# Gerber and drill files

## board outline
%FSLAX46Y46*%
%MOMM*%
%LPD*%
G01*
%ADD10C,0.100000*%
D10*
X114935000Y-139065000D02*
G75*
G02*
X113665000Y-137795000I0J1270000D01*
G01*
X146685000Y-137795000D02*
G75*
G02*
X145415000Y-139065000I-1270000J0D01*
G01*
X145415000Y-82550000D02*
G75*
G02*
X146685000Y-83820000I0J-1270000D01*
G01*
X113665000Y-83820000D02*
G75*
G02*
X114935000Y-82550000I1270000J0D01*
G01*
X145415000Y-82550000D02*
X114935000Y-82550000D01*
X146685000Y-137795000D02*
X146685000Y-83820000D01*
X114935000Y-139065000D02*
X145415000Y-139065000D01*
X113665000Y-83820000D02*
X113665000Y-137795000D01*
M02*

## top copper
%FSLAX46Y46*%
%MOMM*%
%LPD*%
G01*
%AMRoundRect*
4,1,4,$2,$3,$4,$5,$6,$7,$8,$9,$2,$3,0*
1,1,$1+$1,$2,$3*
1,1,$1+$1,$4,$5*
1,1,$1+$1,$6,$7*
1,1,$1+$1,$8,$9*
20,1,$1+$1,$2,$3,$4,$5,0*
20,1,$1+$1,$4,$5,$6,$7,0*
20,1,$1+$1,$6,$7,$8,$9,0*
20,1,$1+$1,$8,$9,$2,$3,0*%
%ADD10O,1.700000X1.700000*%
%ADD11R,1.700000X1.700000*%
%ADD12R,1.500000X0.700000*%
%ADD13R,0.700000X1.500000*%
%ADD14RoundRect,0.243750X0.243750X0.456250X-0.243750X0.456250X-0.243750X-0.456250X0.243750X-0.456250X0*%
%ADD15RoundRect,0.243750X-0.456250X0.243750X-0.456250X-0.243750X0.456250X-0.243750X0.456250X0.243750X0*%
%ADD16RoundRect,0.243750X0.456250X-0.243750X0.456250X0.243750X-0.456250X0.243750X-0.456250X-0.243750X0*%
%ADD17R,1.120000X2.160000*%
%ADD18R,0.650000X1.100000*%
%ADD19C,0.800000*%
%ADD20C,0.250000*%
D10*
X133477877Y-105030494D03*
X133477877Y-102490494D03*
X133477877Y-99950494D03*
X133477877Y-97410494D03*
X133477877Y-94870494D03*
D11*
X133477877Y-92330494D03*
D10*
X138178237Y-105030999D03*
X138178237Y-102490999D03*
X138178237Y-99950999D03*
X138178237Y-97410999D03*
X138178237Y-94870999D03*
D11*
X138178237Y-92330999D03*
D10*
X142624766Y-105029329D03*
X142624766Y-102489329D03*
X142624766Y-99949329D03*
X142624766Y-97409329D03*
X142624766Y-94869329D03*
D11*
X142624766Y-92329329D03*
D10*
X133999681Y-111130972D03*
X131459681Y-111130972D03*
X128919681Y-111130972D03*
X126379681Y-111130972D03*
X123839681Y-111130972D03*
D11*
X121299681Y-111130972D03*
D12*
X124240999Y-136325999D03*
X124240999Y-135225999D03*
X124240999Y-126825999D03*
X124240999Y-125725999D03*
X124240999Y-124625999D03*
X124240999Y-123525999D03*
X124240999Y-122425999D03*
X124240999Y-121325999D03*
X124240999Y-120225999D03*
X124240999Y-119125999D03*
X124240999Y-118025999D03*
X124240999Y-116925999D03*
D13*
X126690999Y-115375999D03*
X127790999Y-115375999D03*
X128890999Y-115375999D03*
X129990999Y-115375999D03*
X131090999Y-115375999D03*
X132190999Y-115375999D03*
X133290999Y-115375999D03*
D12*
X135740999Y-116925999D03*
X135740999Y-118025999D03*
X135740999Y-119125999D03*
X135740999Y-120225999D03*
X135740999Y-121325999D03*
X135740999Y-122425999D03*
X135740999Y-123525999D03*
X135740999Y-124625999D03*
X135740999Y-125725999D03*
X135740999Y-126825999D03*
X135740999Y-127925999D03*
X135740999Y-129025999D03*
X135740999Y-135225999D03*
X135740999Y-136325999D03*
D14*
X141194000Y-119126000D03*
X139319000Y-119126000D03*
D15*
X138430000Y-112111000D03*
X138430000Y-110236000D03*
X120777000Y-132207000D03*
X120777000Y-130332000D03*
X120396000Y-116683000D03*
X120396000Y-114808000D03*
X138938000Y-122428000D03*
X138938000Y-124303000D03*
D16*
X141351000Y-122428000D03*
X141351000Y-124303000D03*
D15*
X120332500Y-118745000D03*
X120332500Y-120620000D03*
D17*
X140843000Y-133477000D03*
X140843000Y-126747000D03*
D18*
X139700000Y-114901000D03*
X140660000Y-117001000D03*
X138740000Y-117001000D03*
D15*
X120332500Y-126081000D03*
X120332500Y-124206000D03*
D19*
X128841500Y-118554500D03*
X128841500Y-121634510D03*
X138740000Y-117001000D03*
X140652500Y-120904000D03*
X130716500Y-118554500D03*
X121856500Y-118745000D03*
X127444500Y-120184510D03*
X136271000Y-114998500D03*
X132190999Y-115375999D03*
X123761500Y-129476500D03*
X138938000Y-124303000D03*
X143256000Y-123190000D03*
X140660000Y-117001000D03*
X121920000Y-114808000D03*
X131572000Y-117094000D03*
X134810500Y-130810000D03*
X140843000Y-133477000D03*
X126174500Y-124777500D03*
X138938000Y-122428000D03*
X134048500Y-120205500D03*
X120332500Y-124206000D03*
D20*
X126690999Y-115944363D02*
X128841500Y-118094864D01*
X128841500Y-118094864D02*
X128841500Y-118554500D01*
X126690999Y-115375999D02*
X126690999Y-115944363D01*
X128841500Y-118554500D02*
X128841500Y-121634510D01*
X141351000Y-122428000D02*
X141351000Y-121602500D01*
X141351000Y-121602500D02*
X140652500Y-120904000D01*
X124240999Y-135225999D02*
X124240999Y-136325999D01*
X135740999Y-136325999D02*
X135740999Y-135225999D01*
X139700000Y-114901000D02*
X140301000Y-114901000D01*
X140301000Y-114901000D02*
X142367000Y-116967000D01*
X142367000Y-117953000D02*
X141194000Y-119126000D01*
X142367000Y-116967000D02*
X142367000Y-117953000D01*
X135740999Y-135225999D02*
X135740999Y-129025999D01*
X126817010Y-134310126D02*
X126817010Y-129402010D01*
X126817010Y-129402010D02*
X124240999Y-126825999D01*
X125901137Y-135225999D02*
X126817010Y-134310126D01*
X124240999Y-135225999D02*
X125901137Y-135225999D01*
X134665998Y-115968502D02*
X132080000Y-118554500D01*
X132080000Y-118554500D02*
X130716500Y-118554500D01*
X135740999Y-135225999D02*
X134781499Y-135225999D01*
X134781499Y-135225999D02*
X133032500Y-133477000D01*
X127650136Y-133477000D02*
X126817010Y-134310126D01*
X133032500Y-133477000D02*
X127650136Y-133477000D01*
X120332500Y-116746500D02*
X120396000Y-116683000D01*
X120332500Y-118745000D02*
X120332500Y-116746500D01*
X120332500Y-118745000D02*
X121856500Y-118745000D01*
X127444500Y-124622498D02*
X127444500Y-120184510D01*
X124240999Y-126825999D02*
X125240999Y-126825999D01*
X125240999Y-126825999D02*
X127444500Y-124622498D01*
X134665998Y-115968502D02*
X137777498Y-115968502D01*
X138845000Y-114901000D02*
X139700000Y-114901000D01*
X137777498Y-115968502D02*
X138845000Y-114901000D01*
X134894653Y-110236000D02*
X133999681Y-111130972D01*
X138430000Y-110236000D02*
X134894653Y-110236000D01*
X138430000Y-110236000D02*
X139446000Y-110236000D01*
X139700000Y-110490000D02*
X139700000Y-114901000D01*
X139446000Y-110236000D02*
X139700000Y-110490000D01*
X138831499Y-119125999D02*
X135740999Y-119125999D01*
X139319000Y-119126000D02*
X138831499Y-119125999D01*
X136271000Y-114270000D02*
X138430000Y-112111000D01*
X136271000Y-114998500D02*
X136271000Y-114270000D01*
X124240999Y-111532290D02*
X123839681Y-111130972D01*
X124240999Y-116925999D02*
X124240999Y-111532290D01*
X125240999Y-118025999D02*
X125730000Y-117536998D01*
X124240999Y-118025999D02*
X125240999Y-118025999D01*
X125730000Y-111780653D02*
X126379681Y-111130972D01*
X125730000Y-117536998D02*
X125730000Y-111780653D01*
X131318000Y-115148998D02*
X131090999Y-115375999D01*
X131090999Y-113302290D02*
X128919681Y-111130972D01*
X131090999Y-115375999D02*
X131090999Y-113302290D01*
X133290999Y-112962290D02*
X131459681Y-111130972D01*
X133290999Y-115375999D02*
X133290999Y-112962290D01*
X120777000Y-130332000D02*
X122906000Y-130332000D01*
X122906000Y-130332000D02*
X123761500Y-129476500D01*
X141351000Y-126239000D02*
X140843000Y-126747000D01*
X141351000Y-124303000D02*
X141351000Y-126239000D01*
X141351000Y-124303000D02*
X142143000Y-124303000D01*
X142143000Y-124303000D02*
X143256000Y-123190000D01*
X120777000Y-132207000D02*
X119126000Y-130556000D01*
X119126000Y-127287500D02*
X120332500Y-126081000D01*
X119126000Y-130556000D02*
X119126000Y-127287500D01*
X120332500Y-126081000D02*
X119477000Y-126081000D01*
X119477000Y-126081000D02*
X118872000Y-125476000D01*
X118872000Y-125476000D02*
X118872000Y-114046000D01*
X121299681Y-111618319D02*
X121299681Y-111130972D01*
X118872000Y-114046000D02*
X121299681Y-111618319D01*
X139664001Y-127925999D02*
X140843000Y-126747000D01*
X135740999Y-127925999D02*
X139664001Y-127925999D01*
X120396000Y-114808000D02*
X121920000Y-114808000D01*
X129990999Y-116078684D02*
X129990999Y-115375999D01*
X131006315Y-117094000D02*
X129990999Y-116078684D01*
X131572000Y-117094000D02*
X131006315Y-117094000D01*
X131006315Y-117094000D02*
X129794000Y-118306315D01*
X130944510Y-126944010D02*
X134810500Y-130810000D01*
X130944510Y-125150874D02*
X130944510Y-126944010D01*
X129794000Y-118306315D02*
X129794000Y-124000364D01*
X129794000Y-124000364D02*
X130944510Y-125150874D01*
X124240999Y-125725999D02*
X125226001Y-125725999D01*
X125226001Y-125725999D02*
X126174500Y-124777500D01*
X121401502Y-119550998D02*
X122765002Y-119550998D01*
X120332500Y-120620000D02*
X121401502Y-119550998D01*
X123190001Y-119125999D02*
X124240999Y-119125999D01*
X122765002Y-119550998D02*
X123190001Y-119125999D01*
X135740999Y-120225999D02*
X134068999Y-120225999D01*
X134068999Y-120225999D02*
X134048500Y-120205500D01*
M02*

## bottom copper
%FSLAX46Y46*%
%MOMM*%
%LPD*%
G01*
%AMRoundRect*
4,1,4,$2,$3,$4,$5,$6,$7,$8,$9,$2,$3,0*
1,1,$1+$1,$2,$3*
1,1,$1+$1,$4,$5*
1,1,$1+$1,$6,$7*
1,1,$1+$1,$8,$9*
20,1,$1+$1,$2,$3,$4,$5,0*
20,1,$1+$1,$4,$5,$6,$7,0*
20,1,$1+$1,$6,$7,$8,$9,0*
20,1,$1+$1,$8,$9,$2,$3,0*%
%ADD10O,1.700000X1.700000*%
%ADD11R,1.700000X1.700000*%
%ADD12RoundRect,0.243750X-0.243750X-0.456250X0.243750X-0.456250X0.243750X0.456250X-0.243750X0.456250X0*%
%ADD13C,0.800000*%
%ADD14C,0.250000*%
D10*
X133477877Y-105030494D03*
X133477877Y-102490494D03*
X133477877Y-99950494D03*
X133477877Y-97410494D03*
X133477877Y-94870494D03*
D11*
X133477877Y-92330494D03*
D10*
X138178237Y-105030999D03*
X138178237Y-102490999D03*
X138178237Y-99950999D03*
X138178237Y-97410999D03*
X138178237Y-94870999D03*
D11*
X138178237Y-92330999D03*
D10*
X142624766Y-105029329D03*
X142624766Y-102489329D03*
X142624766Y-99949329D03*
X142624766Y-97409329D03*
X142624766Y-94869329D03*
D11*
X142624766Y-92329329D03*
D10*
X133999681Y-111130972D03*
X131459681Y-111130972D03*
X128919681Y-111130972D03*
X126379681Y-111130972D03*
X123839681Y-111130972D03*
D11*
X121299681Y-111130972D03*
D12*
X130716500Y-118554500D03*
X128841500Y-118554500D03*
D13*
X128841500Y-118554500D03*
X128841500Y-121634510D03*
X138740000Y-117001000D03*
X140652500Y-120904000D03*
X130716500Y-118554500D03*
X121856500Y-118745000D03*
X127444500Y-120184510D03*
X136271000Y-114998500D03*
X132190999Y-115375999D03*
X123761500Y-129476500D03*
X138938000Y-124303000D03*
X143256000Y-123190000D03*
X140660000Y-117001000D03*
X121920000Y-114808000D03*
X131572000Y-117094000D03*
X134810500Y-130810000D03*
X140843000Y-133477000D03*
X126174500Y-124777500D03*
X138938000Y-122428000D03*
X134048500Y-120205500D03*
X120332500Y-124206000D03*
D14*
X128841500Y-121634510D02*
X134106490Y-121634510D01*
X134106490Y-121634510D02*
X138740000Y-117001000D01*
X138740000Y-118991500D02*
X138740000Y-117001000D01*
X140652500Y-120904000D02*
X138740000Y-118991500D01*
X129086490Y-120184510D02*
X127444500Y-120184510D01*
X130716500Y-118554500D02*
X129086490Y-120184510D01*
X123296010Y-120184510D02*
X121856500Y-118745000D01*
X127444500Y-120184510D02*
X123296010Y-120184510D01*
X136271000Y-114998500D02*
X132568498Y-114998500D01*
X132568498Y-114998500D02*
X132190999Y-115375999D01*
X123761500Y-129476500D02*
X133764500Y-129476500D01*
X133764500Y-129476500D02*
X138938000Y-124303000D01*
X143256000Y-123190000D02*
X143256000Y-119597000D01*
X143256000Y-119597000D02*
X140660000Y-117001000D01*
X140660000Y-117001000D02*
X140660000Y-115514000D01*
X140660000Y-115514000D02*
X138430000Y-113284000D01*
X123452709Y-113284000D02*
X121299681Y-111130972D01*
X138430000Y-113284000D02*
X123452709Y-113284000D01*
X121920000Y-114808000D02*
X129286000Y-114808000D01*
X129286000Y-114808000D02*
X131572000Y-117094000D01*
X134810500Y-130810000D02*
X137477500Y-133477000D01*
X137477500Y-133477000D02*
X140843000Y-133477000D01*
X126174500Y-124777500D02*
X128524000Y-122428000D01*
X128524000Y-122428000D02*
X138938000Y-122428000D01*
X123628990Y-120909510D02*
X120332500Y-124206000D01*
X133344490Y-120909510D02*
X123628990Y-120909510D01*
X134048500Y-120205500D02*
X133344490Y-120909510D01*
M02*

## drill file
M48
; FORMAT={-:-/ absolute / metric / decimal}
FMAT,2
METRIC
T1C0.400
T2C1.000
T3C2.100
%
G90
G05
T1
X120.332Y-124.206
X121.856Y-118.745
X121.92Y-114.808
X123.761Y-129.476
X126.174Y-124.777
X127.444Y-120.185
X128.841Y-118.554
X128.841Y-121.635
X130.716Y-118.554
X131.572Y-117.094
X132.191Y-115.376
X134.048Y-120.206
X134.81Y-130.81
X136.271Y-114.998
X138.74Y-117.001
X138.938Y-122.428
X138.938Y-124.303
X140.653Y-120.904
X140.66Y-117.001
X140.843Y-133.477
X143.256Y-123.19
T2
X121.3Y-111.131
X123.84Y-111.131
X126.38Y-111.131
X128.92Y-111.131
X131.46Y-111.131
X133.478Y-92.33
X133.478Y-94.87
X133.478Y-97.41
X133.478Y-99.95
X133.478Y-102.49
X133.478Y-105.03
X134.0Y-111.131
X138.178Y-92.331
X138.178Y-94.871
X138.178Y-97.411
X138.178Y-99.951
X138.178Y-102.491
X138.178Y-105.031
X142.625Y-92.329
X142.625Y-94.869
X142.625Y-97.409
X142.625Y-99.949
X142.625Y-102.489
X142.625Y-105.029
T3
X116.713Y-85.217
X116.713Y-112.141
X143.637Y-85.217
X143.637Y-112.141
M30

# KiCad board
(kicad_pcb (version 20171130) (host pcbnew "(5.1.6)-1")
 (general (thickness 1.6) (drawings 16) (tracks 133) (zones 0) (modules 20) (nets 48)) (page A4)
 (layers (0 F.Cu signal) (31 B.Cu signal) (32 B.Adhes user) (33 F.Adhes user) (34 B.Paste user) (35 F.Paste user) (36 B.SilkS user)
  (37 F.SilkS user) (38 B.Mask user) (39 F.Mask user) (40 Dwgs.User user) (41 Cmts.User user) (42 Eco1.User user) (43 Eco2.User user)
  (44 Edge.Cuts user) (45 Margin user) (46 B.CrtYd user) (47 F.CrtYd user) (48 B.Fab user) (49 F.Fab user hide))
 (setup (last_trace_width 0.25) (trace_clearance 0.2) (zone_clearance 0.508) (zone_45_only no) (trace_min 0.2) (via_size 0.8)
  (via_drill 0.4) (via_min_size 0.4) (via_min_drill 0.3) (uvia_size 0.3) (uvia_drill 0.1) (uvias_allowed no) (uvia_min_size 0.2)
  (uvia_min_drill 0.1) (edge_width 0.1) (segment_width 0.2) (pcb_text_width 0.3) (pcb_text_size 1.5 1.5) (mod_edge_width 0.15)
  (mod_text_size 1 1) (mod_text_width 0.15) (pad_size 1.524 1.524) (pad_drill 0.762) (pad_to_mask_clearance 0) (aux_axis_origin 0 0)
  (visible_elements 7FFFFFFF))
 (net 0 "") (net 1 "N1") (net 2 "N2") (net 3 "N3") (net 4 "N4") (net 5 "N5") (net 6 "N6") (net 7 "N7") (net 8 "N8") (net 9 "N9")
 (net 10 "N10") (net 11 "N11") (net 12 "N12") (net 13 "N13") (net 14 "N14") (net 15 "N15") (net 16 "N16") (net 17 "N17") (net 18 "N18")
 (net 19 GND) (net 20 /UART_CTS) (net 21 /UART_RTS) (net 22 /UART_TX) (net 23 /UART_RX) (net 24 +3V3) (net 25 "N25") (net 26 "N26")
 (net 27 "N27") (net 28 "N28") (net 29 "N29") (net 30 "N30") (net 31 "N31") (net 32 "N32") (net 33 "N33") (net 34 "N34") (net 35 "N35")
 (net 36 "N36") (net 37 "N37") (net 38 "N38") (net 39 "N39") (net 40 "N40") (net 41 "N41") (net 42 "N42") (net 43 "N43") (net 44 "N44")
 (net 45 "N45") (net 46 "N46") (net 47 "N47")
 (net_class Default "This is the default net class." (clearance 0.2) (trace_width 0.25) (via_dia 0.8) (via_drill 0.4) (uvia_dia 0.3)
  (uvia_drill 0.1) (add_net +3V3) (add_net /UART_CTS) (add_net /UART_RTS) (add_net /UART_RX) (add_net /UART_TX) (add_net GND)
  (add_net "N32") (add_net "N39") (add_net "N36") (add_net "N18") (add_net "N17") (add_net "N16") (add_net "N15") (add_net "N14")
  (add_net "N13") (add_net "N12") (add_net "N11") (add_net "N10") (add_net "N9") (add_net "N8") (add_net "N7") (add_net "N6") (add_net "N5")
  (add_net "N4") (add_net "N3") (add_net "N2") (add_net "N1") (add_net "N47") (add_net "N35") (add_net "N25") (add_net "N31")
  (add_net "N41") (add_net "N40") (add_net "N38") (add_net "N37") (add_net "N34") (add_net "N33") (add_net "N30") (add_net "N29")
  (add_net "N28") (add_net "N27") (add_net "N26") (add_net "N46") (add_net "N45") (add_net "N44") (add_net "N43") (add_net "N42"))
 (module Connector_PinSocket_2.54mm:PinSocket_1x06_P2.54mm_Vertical (layer B.Cu) (at 133.477877 92.330494 180)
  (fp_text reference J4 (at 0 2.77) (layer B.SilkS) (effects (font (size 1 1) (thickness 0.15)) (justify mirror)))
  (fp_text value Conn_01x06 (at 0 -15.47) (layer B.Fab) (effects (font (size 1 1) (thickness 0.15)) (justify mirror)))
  (pad 6 thru_hole oval (at 0 -12.7 180) (size 1.7 1.7) (drill 1) (layers *.Cu *.Mask) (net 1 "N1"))
  (pad 5 thru_hole oval (at 0 -10.16 180) (size 1.7 1.7) (drill 1) (layers *.Cu *.Mask) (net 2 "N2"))
  (pad 4 thru_hole oval (at 0 -7.62 180) (size 1.7 1.7) (drill 1) (layers *.Cu *.Mask) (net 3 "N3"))
  (pad 3 thru_hole oval (at 0 -5.08 180) (size 1.7 1.7) (drill 1) (layers *.Cu *.Mask) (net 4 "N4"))
  (pad 2 thru_hole oval (at 0 -2.54 180) (size 1.7 1.7) (drill 1) (layers *.Cu *.Mask) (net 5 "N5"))
  (pad 1 thru_hole rect (at 0 0 180) (size 1.7 1.7) (drill 1) (layers *.Cu *.Mask) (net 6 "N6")))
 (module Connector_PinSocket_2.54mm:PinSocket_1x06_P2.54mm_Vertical (layer B.Cu) (at 138.178237 92.330999 180)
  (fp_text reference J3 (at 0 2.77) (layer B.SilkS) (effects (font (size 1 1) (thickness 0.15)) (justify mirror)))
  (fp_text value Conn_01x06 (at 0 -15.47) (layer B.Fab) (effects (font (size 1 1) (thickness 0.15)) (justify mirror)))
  (pad 6 thru_hole oval (at 0 -12.7 180) (size 1.7 1.7) (drill 1) (layers *.Cu *.Mask) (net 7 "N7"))
  (pad 5 thru_hole oval (at 0 -10.16 180) (size 1.7 1.7) (drill 1) (layers *.Cu *.Mask) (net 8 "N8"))
  (pad 4 thru_hole oval (at 0 -7.62 180) (size 1.7 1.7) (drill 1) (layers *.Cu *.Mask) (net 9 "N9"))
  (pad 3 thru_hole oval (at 0 -5.08 180) (size 1.7 1.7) (drill 1) (layers *.Cu *.Mask) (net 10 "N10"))
  (pad 2 thru_hole oval (at 0 -2.54 180) (size 1.7 1.7) (drill 1) (layers *.Cu *.Mask) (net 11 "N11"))
  (pad 1 thru_hole rect (at 0 0 180) (size 1.7 1.7) (drill 1) (layers *.Cu *.Mask) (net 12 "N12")))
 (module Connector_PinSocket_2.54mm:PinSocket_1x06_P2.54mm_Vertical (layer B.Cu) (at 142.624766 92.329329 180)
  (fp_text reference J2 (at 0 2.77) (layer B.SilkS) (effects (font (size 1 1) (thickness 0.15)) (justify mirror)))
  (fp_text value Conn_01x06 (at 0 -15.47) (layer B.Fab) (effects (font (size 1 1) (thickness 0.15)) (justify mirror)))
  (pad 6 thru_hole oval (at 0 -12.7 180) (size 1.7 1.7) (drill 1) (layers *.Cu *.Mask) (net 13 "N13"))
  (pad 5 thru_hole oval (at 0 -10.16 180) (size 1.7 1.7) (drill 1) (layers *.Cu *.Mask) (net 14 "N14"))
  (pad 4 thru_hole oval (at 0 -7.62 180) (size 1.7 1.7) (drill 1) (layers *.Cu *.Mask) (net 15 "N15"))
  (pad 3 thru_hole oval (at 0 -5.08 180) (size 1.7 1.7) (drill 1) (layers *.Cu *.Mask) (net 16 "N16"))
  (pad 2 thru_hole oval (at 0 -2.54 180) (size 1.7 1.7) (drill 1) (layers *.Cu *.Mask) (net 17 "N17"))
  (pad 1 thru_hole rect (at 0 0 180) (size 1.7 1.7) (drill 1) (layers *.Cu *.Mask) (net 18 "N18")))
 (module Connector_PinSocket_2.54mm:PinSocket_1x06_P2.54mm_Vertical (layer B.Cu) (at 121.299681 111.130972 270)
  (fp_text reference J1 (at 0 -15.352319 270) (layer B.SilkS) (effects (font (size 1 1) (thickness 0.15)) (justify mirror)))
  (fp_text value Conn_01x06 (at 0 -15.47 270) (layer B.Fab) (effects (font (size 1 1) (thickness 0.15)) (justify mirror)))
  (pad 6 thru_hole oval (at 0 -12.7 270) (size 1.7 1.7) (drill 1) (layers *.Cu *.Mask) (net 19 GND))
  (pad 5 thru_hole oval (at 0 -10.16 270) (size 1.7 1.7) (drill 1) (layers *.Cu *.Mask) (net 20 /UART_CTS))
  (pad 4 thru_hole oval (at 0 -7.62 270) (size 1.7 1.7) (drill 1) (layers *.Cu *.Mask) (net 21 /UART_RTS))
  (pad 3 thru_hole oval (at 0 -5.08 270) (size 1.7 1.7) (drill 1) (layers *.Cu *.Mask) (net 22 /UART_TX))
  (pad 2 thru_hole oval (at 0 -2.54 270) (size 1.7 1.7) (drill 1) (layers *.Cu *.Mask) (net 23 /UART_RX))
  (pad 1 thru_hole rect (at 0 0 270) (size 1.7 1.7) (drill 1) (layers *.Cu *.Mask) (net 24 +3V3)))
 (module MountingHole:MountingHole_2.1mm (layer F.Cu) (at 143.637 112.141)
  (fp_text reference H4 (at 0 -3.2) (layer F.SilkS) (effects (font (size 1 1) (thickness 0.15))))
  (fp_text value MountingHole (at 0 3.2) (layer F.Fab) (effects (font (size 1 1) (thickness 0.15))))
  (pad "" np_thru_hole circle (at 0 0) (size 2.1 2.1) (drill 2.1) (layers *.Cu *.Mask)))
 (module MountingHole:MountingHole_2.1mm (layer F.Cu) (at 116.713 112.141)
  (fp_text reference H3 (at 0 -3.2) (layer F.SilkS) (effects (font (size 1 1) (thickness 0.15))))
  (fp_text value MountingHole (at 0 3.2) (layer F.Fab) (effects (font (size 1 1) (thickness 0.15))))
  (pad "" np_thru_hole circle (at 0 0) (size 2.1 2.1) (drill 2.1) (layers *.Cu *.Mask)))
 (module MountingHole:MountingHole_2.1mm (layer F.Cu) (at 143.637 85.217)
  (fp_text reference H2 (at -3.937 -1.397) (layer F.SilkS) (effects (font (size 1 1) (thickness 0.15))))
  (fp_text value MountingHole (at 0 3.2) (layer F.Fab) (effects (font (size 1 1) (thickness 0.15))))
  (pad "" np_thru_hole circle (at 0 0) (size 2.1 2.1) (drill 2.1) (layers *.Cu *.Mask)))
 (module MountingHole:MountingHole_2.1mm (layer F.Cu) (at 116.713 85.217)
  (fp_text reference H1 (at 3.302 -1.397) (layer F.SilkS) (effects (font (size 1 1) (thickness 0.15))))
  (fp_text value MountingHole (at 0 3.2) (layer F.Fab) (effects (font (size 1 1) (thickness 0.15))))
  (pad "" np_thru_hole circle (at 0 0) (size 2.1 2.1) (drill 2.1) (layers *.Cu *.Mask)))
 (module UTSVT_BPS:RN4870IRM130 (layer F.Cu) (at 129.990999 126.125999 180)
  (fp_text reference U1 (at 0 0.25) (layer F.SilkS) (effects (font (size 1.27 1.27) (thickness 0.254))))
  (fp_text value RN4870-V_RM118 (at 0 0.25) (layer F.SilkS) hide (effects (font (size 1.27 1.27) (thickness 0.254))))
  (pad 33 smd rect (at 5.75 -10.2 270) (size 0.7 1.5) (layers F.Cu F.Paste F.Mask) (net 19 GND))
  (pad 32 smd rect (at 5.75 -9.1 270) (size 0.7 1.5) (layers F.Cu F.Paste F.Mask) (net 19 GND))
  (pad 31 smd rect (at 5.75 -0.7 270) (size 0.7 1.5) (layers F.Cu F.Paste F.Mask) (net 19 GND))
  (pad 30 smd rect (at 5.75 0.4 270) (size 0.7 1.5) (layers F.Cu F.Paste F.Mask) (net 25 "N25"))
  (pad 29 smd rect (at 5.75 1.5 270) (size 0.7 1.5) (layers F.Cu F.Paste F.Mask) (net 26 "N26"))
  (pad 28 smd rect (at 5.75 2.6 270) (size 0.7 1.5) (layers F.Cu F.Paste F.Mask) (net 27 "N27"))
  (pad 27 smd rect (at 5.75 3.7 270) (size 0.7 1.5) (layers F.Cu F.Paste F.Mask) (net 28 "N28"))
  (pad 26 smd rect (at 5.75 4.8 270) (size 0.7 1.5) (layers F.Cu F.Paste F.Mask) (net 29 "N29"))
  (pad 25 smd rect (at 5.75 5.9 270) (size 0.7 1.5) (layers F.Cu F.Paste F.Mask) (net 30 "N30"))
  (pad 24 smd rect (at 5.75 7 270) (size 0.7 1.5) (layers F.Cu F.Paste F.Mask) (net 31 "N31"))
  (pad 23 smd rect (at 5.75 8.1 270) (size 0.7 1.5) (layers F.Cu F.Paste F.Mask) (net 22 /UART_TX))
  (pad 22 smd rect (at 5.75 9.2 270) (size 0.7 1.5) (layers F.Cu F.Paste F.Mask) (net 23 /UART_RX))
  (pad 21 smd rect (at 3.3 10.75 180) (size 0.7 1.5) (layers F.Cu F.Paste F.Mask) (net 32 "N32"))
  (pad 20 smd rect (at 2.2 10.75 180) (size 0.7 1.5) (layers F.Cu F.Paste F.Mask) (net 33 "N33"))
  (pad 19 smd rect (at 1.1 10.75 180) (size 0.7 1.5) (layers F.Cu F.Paste F.Mask) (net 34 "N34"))
  (pad 18 smd rect (at 0 10.75 180) (size 0.7 1.5) (layers F.Cu F.Paste F.Mask) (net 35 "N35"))
  (pad 17 smd rect (at -1.1 10.75 180) (size 0.7 1.5) (layers F.Cu F.Paste F.Mask) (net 21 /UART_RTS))
  (pad 16 smd rect (at -2.2 10.75 180) (size 0.7 1.5) (layers F.Cu F.Paste F.Mask) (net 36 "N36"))
  (pad 15 smd rect (at -3.3 10.75 180) (size 0.7 1.5) (layers F.Cu F.Paste F.Mask) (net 20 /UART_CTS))
  (pad 14 smd rect (at -5.75 9.2 270) (size 0.7 1.5) (layers F.Cu F.Paste F.Mask) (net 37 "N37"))
  (pad 13 smd rect (at -5.75 8.1 270) (size 0.7 1.5) (layers F.Cu F.Paste F.Mask) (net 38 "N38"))
  (pad 12 smd rect (at -5.75 7 270) (size 0.7 1.5) (layers F.Cu F.Paste F.Mask) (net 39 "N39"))
  (pad 11 smd rect (at -5.75 5.9 270) (size 0.7 1.5) (layers F.Cu F.Paste F.Mask) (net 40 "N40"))
  (pad 10 smd rect (at -5.75 4.8 270) (size 0.7 1.5) (layers F.Cu F.Paste F.Mask) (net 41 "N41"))
  (pad 9 smd rect (at -5.75 3.7 270) (size 0.7 1.5) (layers F.Cu F.Paste F.Mask) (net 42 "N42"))
  (pad 8 smd rect (at -5.75 2.6 270) (size 0.7 1.5) (layers F.Cu F.Paste F.Mask) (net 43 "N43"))
  (pad 7 smd rect (at -5.75 1.5 270) (size 0.7 1.5) (layers F.Cu F.Paste F.Mask) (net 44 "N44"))
  (pad 6 smd rect (at -5.75 0.4 270) (size 0.7 1.5) (layers F.Cu F.Paste F.Mask) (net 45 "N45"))
  (pad 5 smd rect (at -5.75 -0.7 270) (size 0.7 1.5) (layers F.Cu F.Paste F.Mask) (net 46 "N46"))
  (pad 4 smd rect (at -5.75 -1.8 270) (size 0.7 1.5) (layers F.Cu F.Paste F.Mask) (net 24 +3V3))
  (pad 3 smd rect (at -5.75 -2.9 270) (size 0.7 1.5) (layers F.Cu F.Paste F.Mask) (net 19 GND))
  (pad 2 smd rect (at -5.75 -9.1 270) (size 0.7 1.5) (layers F.Cu F.Paste F.Mask) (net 19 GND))
  (pad 1 smd rect (at -5.75 -10.2 270) (size 0.7 1.5) (layers F.Cu F.Paste F.Mask) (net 19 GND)))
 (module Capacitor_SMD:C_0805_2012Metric (layer B.Cu) (at 129.779 118.5545)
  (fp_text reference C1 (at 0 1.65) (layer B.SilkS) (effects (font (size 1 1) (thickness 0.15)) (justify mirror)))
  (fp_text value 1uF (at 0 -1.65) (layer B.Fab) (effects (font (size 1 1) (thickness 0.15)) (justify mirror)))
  (pad 2 smd roundrect (at 0.9375 0) (size 0.975 1.4) (layers B.Cu B.Paste B.Mask) (roundrect_rratio 0.25) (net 19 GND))
  (pad 1 smd roundrect (at -0.9375 0) (size 0.975 1.4) (layers B.Cu B.Paste B.Mask) (roundrect_rratio 0.25) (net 32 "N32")))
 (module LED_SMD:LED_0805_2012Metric (layer F.Cu) (at 140.2565 119.126 180)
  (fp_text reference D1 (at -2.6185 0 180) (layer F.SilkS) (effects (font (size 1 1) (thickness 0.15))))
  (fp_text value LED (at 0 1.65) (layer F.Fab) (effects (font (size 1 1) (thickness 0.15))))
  (pad 1 smd roundrect (at -0.9375 0 180) (size 0.975 1.4) (layers F.Cu F.Paste F.Mask) (roundrect_rratio 0.25) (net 19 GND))
  (pad 2 smd roundrect (at 0.9375 0 180) (size 0.975 1.4) (layers F.Cu F.Paste F.Mask) (roundrect_rratio 0.25) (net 39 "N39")))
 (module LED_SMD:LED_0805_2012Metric (layer F.Cu) (at 138.43 111.1735 270)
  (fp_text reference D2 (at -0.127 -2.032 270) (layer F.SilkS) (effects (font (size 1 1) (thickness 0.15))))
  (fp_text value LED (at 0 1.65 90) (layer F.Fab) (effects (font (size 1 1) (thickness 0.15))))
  (pad 2 smd roundrect (at 0.9375 0 270) (size 0.975 1.4) (layers F.Cu F.Paste F.Mask) (roundrect_rratio 0.25) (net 36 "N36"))
  (pad 1 smd roundrect (at -0.9375 0 270) (size 0.975 1.4) (layers F.Cu F.Paste F.Mask) (roundrect_rratio 0.25) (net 19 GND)))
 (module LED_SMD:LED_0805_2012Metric (layer F.Cu) (at 120.777 131.2695 270)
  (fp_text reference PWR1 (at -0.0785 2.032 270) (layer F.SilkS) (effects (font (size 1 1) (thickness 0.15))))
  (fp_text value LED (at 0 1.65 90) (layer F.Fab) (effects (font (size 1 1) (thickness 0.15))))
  (pad 2 smd roundrect (at 0.9375 0 270) (size 0.975 1.4) (layers F.Cu F.Paste F.Mask) (roundrect_rratio 0.25) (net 24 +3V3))
  (pad 1 smd roundrect (at -0.9375 0 270) (size 0.975 1.4) (layers F.Cu F.Paste F.Mask) (roundrect_rratio 0.25) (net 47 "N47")))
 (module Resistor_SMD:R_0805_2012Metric (layer F.Cu) (at 120.396 115.7455 270)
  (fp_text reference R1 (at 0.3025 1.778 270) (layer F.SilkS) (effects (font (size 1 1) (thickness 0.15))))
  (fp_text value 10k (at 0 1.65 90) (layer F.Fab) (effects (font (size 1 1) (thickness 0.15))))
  (pad 2 smd roundrect (at 0.9375 0 270) (size 0.975 1.4) (layers F.Cu F.Paste F.Mask) (roundrect_rratio 0.25) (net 19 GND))
  (pad 1 smd roundrect (at -0.9375 0 270) (size 0.975 1.4) (layers F.Cu F.Paste F.Mask) (roundrect_rratio 0.25) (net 35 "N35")))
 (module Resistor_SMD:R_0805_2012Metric (layer F.Cu) (at 138.938 123.3655 270)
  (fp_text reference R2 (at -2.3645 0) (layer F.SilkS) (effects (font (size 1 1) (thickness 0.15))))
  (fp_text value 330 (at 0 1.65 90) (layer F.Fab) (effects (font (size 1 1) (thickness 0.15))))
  (pad 1 smd roundrect (at -0.9375 0 270) (size 0.975 1.4) (layers F.Cu F.Paste F.Mask) (roundrect_rratio 0.25) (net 25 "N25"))
  (pad 2 smd roundrect (at 0.9375 0 270) (size 0.975 1.4) (layers F.Cu F.Paste F.Mask) (roundrect_rratio 0.25) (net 47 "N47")))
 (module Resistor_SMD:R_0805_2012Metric (layer F.Cu) (at 141.351 123.3655 90)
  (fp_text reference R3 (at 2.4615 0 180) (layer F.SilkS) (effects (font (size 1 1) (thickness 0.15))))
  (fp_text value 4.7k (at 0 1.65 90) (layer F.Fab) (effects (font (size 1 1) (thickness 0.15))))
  (pad 2 smd roundrect (at 0.9375 0 90) (size 0.975 1.4) (layers F.Cu F.Paste F.Mask) (roundrect_rratio 0.25) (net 32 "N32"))
  (pad 1 smd roundrect (at -0.9375 0 90) (size 0.975 1.4) (layers F.Cu F.Paste F.Mask) (roundrect_rratio 0.25) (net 24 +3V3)))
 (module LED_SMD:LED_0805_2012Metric (layer F.Cu) (at 120.3325 119.6825 270)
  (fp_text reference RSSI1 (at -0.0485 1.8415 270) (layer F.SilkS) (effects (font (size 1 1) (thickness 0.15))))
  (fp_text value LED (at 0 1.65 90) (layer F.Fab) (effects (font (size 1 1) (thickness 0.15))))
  (pad 1 smd roundrect (at -0.9375 0 270) (size 0.975 1.4) (layers F.Cu F.Paste F.Mask) (roundrect_rratio 0.25) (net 19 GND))
  (pad 2 smd roundrect (at 0.9375 0 270) (size 0.975 1.4) (layers F.Cu F.Paste F.Mask) (roundrect_rratio 0.25) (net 31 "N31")))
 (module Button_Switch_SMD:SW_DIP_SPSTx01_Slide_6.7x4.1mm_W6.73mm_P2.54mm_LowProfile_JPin (layer F.Cu) (at 140.843 130.112 270)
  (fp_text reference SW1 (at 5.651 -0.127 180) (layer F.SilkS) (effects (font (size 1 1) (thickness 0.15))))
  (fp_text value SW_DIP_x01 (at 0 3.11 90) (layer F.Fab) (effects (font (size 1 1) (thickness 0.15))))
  (pad 2 smd rect (at 3.365 0 270) (size 2.16 1.12) (layers F.Cu F.Paste F.Mask) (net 35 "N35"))
  (pad 1 smd rect (at -3.365 0 270) (size 2.16 1.12) (layers F.Cu F.Paste F.Mask) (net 24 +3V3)))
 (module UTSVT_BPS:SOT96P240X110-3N (layer F.Cu) (at 139.7 115.951 90)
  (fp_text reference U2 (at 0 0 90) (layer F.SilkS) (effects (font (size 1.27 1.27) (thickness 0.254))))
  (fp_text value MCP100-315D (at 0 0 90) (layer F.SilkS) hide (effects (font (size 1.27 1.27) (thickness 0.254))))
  (pad 3 smd rect (at 1.05 0 180) (size 0.65 1.1) (layers F.Cu F.Paste F.Mask) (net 19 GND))
  (pad 2 smd rect (at -1.05 0.96 180) (size 0.65 1.1) (layers F.Cu F.Paste F.Mask) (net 24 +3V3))
  (pad 1 smd rect (at -1.05 -0.96 180) (size 0.65 1.1) (layers F.Cu F.Paste F.Mask) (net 32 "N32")))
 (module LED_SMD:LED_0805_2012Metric (layer F.Cu) (at 120.3325 125.1435 270)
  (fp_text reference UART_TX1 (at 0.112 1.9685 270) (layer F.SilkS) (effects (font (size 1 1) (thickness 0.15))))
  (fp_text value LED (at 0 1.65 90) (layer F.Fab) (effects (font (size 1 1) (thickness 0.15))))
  (pad 2 smd roundrect (at 0.9375 0 270) (size 0.975 1.4) (layers F.Cu F.Paste F.Mask) (roundrect_rratio 0.25) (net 24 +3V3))
  (pad 1 smd roundrect (at -0.9375 0 270) (size 0.975 1.4) (layers F.Cu F.Paste F.Mask) (roundrect_rratio 0.25) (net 40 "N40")))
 (gr_arc (start 114.935 137.795) (end 113.665 137.795) (angle -90) (layer Edge.Cuts) (width 0.1))
 (gr_arc (start 145.415 137.795) (end 145.415 139.065) (angle -90) (layer Edge.Cuts) (width 0.1))
 (gr_arc (start 145.415 83.82) (end 146.685 83.82) (angle -90) (layer Edge.Cuts) (width 0.1))
 (gr_arc (start 114.935 83.82) (end 114.935 82.55) (angle -90) (layer Edge.Cuts) (width 0.1))
 (gr_line (start 145.415 82.55) (end 114.935 82.55) (layer Edge.Cuts) (width 0.1))
 (gr_line (start 146.685 137.795) (end 146.685 83.82) (layer Edge.Cuts) (width 0.1))
 (gr_line (start 114.935 139.065) (end 145.415 139.065) (layer Edge.Cuts) (width 0.1))
 (gr_line (start 113.665 83.82) (end 113.665 137.795) (layer Edge.Cuts) (width 0.1))
 (via (at 128.8415 118.5545) (size 0.8) (drill 0.4) (layers F.Cu B.Cu) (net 32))
 (segment (start 126.690999 115.944363) (end 128.8415 118.094864) (width 0.25) (layer F.Cu) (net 32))
 (segment (start 128.8415 118.094864) (end 128.8415 118.5545) (width 0.25) (layer F.Cu) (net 32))
 (segment (start 126.690999 115.375999) (end 126.690999 115.944363) (width 0.25) (layer F.Cu) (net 32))
 (via (at 128.8415 121.63451) (size 0.8) (drill 0.4) (layers F.Cu B.Cu) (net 32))
 (segment (start 128.8415 118.5545) (end 128.8415 121.63451) (width 0.25) (layer F.Cu) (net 32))
 (via (at 138.74 117.001) (size 0.8) (drill 0.4) (layers F.Cu B.Cu) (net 32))
 (segment (start 128.8415 121.63451) (end 134.10649 121.63451) (width 0.25) (layer B.Cu) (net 32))
 (segment (start 134.10649 121.63451) (end 138.74 117.001) (width 0.25) (layer B.Cu) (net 32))
 (segment (start 141.351 122.428) (end 141.351 121.6025) (width 0.25) (layer F.Cu) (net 32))
 (via (at 140.6525 120.904) (size 0.8) (drill 0.4) (layers F.Cu B.Cu) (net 32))
 (segment (start 141.351 121.6025) (end 140.6525 120.904) (width 0.25) (layer F.Cu) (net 32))
 (segment (start 138.74 118.9915) (end 138.74 117.001) (width 0.25) (layer B.Cu) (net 32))
 (segment (start 140.6525 120.904) (end 138.74 118.9915) (width 0.25) (layer B.Cu) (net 32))
 (segment (start 124.240999 135.225999) (end 124.240999 136.325999) (width 0.25) (layer F.Cu) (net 19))
 (segment (start 135.740999 136.325999) (end 135.740999 135.225999) (width 0.25) (layer F.Cu) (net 19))
 (segment (start 139.7 114.901) (end 140.301 114.901) (width 0.25) (layer F.Cu) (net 19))
 (segment (start 140.301 114.901) (end 142.367 116.967) (width 0.25) (layer F.Cu) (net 19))
 (segment (start 142.367 117.953) (end 141.194 119.126) (width 0.25) (layer F.Cu) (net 19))
 (segment (start 142.367 116.967) (end 142.367 117.953) (width 0.25) (layer F.Cu) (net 19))
 (segment (start 135.740999 135.225999) (end 135.740999 129.025999) (width 0.25) (layer F.Cu) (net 19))
 (segment (start 126.81701 134.310126) (end 126.81701 129.40201) (width 0.25) (layer F.Cu) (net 19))
 (segment (start 126.81701 129.40201) (end 124.240999 126.825999) (width 0.25) (layer F.Cu) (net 19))
 (segment (start 125.901137 135.225999) (end 126.81701 134.310126) (width 0.25) (layer F.Cu) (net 19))
 (segment (start 124.240999 135.225999) (end 125.901137 135.225999) (width 0.25) (layer F.Cu) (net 19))
 (via (at 130.7165 118.5545) (size 0.8) (drill 0.4) (layers F.Cu B.Cu) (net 19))
 (segment (start 134.665998 115.968502) (end 132.08 118.5545) (width 0.25) (layer F.Cu) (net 19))
 (segment (start 132.08 118.5545) (end 130.7165 118.5545) (width 0.25) (layer F.Cu) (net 19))
 (segment (start 135.740999 135.225999) (end 134.781499 135.225999) (width 0.25) (layer F.Cu) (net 19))
 (segment (start 134.781499 135.225999) (end 133.0325 133.477) (width 0.25) (layer F.Cu) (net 19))
 (segment (start 127.650136 133.477) (end 126.81701 134.310126) (width 0.25) (layer F.Cu) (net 19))
 (segment (start 133.0325 133.477) (end 127.650136 133.477) (width 0.25) (layer F.Cu) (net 19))
 (segment (start 120.3325 116.7465) (end 120.396 116.683) (width 0.25) (layer F.Cu) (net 19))
 (segment (start 120.3325 118.745) (end 120.3325 116.7465) (width 0.25) (layer F.Cu) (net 19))
 (via (at 121.8565 118.745) (size 0.8) (drill 0.4) (layers F.Cu B.Cu) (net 19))
 (segment (start 120.3325 118.745) (end 121.8565 118.745) (width 0.25) (layer F.Cu) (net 19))
 (via (at 127.4445 120.18451) (size 0.8) (drill 0.4) (layers F.Cu B.Cu) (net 19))
 (segment (start 127.4445 124.622498) (end 127.4445 120.18451) (width 0.25) (layer F.Cu) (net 19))
 (segment (start 124.240999 126.825999) (end 125.240999 126.825999) (width 0.25) (layer F.Cu) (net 19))
 (segment (start 125.240999 126.825999) (end 127.4445 124.622498) (width 0.25) (layer F.Cu) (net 19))
 (segment (start 129.08649 120.18451) (end 127.4445 120.18451) (width 0.25) (layer B.Cu) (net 19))
 (segment (start 130.7165 118.5545) (end 129.08649 120.18451) (width 0.25) (layer B.Cu) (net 19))
 (segment (start 123.29601 120.18451) (end 121.8565 118.745) (width 0.25) (layer B.Cu) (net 19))
 (segment (start 127.4445 120.18451) (end 123.29601 120.18451) (width 0.25) (layer B.Cu) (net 19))
 (segment (start 134.665998 115.968502) (end 137.777498 115.968502) (width 0.25) (layer F.Cu) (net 19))
 (segment (start 138.845 114.901) (end 139.7 114.901) (width 0.25) (layer F.Cu) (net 19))
 (segment (start 137.777498 115.968502) (end 138.845 114.901) (width 0.25) (layer F.Cu) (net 19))
 (segment (start 134.894653 110.236) (end 133.999681 111.130972) (width 0.25) (layer F.Cu) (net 19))
 (segment (start 138.43 110.236) (end 134.894653 110.236) (width 0.25) (layer F.Cu) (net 19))
 (segment (start 138.43 110.236) (end 139.446 110.236) (width 0.25) (layer F.Cu) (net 19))
 (segment (start 139.7 110.49) (end 139.7 114.901) (width 0.25) (layer F.Cu) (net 19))
 (segment (start 139.446 110.236) (end 139.7 110.49) (width 0.25) (layer F.Cu) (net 19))
 (segment (start 138.831499 119.125999) (end 135.740999 119.125999) (width 0.25) (layer F.Cu) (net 39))
 (segment (start 139.319 119.126) (end 138.831499 119.125999) (width 0.25) (layer F.Cu) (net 39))
 (via (at 136.271 114.9985) (size 0.8) (drill 0.4) (layers F.Cu B.Cu) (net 36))
 (via (at 132.190999 115.375999) (size 0.8) (drill 0.4) (layers F.Cu B.Cu) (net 36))
 (segment (start 136.271 114.9985) (end 132.568498 114.9985) (width 0.25) (layer B.Cu) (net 36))
 (segment (start 132.568498 114.9985) (end 132.190999 115.375999) (width 0.25) (layer B.Cu) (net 36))
 (segment (start 136.271 114.27) (end 138.43 112.111) (width 0.25) (layer F.Cu) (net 36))
 (segment (start 136.271 114.9985) (end 136.271 114.27) (width 0.25) (layer F.Cu) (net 36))
 (segment (start 124.240999 111.53229) (end 123.839681 111.130972) (width 0.25) (layer F.Cu) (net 23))
 (segment (start 124.240999 116.925999) (end 124.240999 111.53229) (width 0.25) (layer F.Cu) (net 23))
 (segment (start 125.240999 118.025999) (end 125.73 117.536998) (width 0.25) (layer F.Cu) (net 22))
 (segment (start 124.240999 118.025999) (end 125.240999 118.025999) (width 0.25) (layer F.Cu) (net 22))
 (segment (start 125.73 111.780653) (end 126.379681 111.130972) (width 0.25) (layer F.Cu) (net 22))
 (segment (start 125.73 117.536998) (end 125.73 111.780653) (width 0.25) (layer F.Cu) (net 22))
 (segment (start 131.318 115.148998) (end 131.090999 115.375999) (width 0.25) (layer F.Cu) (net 21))
 (segment (start 131.090999 113.30229) (end 128.919681 111.130972) (width 0.25) (layer F.Cu) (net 21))
 (segment (start 131.090999 115.375999) (end 131.090999 113.30229) (width 0.25) (layer F.Cu) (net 21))
 (segment (start 133.290999 112.96229) (end 131.459681 111.130972) (width 0.25) (layer F.Cu) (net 20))
 (segment (start 133.290999 115.375999) (end 133.290999 112.96229) (width 0.25) (layer F.Cu) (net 20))
 (via (at 123.7615 129.4765) (size 0.8) (drill 0.4) (layers F.Cu B.Cu) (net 47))
 (segment (start 120.777 130.332) (end 122.906 130.332) (width 0.25) (layer F.Cu) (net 47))
 (segment (start 122.906 130.332) (end 123.7615 129.4765) (width 0.25) (layer F.Cu) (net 47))
 (via (at 138.938 124.303) (size 0.8) (drill 0.4) (layers F.Cu B.Cu) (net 47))
 (segment (start 123.7615 129.4765) (end 133.7645 129.4765) (width 0.25) (layer B.Cu) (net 47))
 (segment (start 133.7645 129.4765) (end 138.938 124.303) (width 0.25) (layer B.Cu) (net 47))
 (segment (start 141.351 126.239) (end 140.843 126.747) (width 0.25) (layer F.Cu) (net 24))
 (segment (start 141.351 124.303) (end 141.351 126.239) (width 0.25) (layer F.Cu) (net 24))
 (via (at 143.256 123.19) (size 0.8) (drill 0.4) (layers F.Cu B.Cu) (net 24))
 (segment (start 141.351 124.303) (end 142.143 124.303) (width 0.25) (layer F.Cu) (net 24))
 (segment (start 142.143 124.303) (end 143.256 123.19) (width 0.25) (layer F.Cu) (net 24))
 (segment (start 120.777 132.207) (end 119.126 130.556) (width 0.25) (layer F.Cu) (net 24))
 (segment (start 119.126 127.2875) (end 120.3325 126.081) (width 0.25) (layer F.Cu) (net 24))
 (segment (start 119.126 130.556) (end 119.126 127.2875) (width 0.25) (layer F.Cu) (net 24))
 (via (at 140.66 117.001) (size 0.8) (drill 0.4) (layers F.Cu B.Cu) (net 24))
 (segment (start 143.256 123.19) (end 143.256 119.597) (width 0.25) (layer B.Cu) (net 24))
 (segment (start 143.256 119.597) (end 140.66 117.001) (width 0.25) (layer B.Cu) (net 24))
 (segment (start 140.66 117.001) (end 140.66 115.514) (width 0.25) (layer B.Cu) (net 24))
 (segment (start 140.66 115.514) (end 138.43 113.284) (width 0.25) (layer B.Cu) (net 24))
 (segment (start 123.452709 113.284) (end 121.299681 111.130972) (width 0.25) (layer B.Cu) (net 24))
 (segment (start 138.43 113.284) (end 123.452709 113.284) (width 0.25) (layer B.Cu) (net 24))
 (segment (start 120.3325 126.081) (end 119.477 126.081) (width 0.25) (layer F.Cu) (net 24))
 (segment (start 119.477 126.081) (end 118.872 125.476) (width 0.25) (layer F.Cu) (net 24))
 (segment (start 118.872 125.476) (end 118.872 114.046) (width 0.25) (layer F.Cu) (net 24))
 (segment (start 121.299681 111.618319) (end 121.299681 111.130972) (width 0.25) (layer F.Cu) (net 24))
 (segment (start 118.872 114.046) (end 121.299681 111.618319) (width 0.25) (layer F.Cu) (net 24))
 (segment (start 139.664001 127.925999) (end 140.843 126.747) (width 0.25) (layer F.Cu) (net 24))
 (segment (start 135.740999 127.925999) (end 139.664001 127.925999) (width 0.25) (layer F.Cu) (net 24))
 (via (at 121.92 114.808) (size 0.8) (drill 0.4) (layers F.Cu B.Cu) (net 35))
 (segment (start 120.396 114.808) (end 121.92 114.808) (width 0.25) (layer F.Cu) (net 35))
 (via (at 131.572 117.094) (size 0.8) (drill 0.4) (layers F.Cu B.Cu) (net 35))
 (segment (start 121.92 114.808) (end 129.286 114.808) (width 0.25) (layer B.Cu) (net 35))
 (segment (start 129.286 114.808) (end 131.572 117.094) (width 0.25) (layer B.Cu) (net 35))
 (segment (start 129.990999 116.078684) (end 129.990999 115.375999) (width 0.25) (layer F.Cu) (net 35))
 (segment (start 131.006315 117.094) (end 129.990999 116.078684) (width 0.25) (layer F.Cu) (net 35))
 (segment (start 131.572 117.094) (end 131.006315 117.094) (width 0.25) (layer F.Cu) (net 35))
 (segment (start 131.006315 117.094) (end 129.794 118.306315) (width 0.25) (layer F.Cu) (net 35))
 (via (at 134.8105 130.81) (size 0.8) (drill 0.4) (layers F.Cu B.Cu) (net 35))
 (segment (start 130.94451 126.94401) (end 134.8105 130.81) (width 0.25) (layer F.Cu) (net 35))
 (segment (start 130.94451 125.150874) (end 130.94451 126.94401) (width 0.25) (layer F.Cu) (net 35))
 (segment (start 129.794 118.306315) (end 129.794 124.000364) (width 0.25) (layer F.Cu) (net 35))
 (segment (start 129.794 124.000364) (end 130.94451 125.150874) (width 0.25) (layer F.Cu) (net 35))
 (via (at 140.843 133.477) (size 0.8) (drill 0.4) (layers F.Cu B.Cu) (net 35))
 (segment (start 134.8105 130.81) (end 137.4775 133.477) (width 0.25) (layer B.Cu) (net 35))
 (segment (start 137.4775 133.477) (end 140.843 133.477) (width 0.25) (layer B.Cu) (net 35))
 (via (at 126.1745 124.7775) (size 0.8) (drill 0.4) (layers F.Cu B.Cu) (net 25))
 (segment (start 124.240999 125.725999) (end 125.226001 125.725999) (width 0.25) (layer F.Cu) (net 25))
 (segment (start 125.226001 125.725999) (end 126.1745 124.7775) (width 0.25) (layer F.Cu) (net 25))
 (via (at 138.938 122.428) (size 0.8) (drill 0.4) (layers F.Cu B.Cu) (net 25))
 (segment (start 126.1745 124.7775) (end 128.524 122.428) (width 0.25) (layer B.Cu) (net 25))
 (segment (start 128.524 122.428) (end 138.938 122.428) (width 0.25) (layer B.Cu) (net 25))
 (segment (start 121.401502 119.550998) (end 122.765002 119.550998) (width 0.25) (layer F.Cu) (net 31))
 (segment (start 120.3325 120.62) (end 121.401502 119.550998) (width 0.25) (layer F.Cu) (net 31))
 (segment (start 123.190001 119.125999) (end 124.240999 119.125999) (width 0.25) (layer F.Cu) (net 31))
 (segment (start 122.765002 119.550998) (end 123.190001 119.125999) (width 0.25) (layer F.Cu) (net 31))
 (via (at 134.0485 120.2055) (size 0.8) (drill 0.4) (layers F.Cu B.Cu) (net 40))
 (segment (start 135.740999 120.225999) (end 134.068999 120.225999) (width 0.25) (layer F.Cu) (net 40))
 (segment (start 134.068999 120.225999) (end 134.0485 120.2055) (width 0.25) (layer F.Cu) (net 40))
 (via (at 120.3325 124.206) (size 0.8) (drill 0.4) (layers F.Cu B.Cu) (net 40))
 (segment (start 123.62899 120.90951) (end 120.3325 124.206) (width 0.25) (layer B.Cu) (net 40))
 (segment (start 133.34449 120.90951) (end 123.62899 120.90951) (width 0.25) (layer B.Cu) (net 40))
 (segment (start 134.0485 120.2055) (end 133.34449 120.90951) (width 0.25) (layer B.Cu) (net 40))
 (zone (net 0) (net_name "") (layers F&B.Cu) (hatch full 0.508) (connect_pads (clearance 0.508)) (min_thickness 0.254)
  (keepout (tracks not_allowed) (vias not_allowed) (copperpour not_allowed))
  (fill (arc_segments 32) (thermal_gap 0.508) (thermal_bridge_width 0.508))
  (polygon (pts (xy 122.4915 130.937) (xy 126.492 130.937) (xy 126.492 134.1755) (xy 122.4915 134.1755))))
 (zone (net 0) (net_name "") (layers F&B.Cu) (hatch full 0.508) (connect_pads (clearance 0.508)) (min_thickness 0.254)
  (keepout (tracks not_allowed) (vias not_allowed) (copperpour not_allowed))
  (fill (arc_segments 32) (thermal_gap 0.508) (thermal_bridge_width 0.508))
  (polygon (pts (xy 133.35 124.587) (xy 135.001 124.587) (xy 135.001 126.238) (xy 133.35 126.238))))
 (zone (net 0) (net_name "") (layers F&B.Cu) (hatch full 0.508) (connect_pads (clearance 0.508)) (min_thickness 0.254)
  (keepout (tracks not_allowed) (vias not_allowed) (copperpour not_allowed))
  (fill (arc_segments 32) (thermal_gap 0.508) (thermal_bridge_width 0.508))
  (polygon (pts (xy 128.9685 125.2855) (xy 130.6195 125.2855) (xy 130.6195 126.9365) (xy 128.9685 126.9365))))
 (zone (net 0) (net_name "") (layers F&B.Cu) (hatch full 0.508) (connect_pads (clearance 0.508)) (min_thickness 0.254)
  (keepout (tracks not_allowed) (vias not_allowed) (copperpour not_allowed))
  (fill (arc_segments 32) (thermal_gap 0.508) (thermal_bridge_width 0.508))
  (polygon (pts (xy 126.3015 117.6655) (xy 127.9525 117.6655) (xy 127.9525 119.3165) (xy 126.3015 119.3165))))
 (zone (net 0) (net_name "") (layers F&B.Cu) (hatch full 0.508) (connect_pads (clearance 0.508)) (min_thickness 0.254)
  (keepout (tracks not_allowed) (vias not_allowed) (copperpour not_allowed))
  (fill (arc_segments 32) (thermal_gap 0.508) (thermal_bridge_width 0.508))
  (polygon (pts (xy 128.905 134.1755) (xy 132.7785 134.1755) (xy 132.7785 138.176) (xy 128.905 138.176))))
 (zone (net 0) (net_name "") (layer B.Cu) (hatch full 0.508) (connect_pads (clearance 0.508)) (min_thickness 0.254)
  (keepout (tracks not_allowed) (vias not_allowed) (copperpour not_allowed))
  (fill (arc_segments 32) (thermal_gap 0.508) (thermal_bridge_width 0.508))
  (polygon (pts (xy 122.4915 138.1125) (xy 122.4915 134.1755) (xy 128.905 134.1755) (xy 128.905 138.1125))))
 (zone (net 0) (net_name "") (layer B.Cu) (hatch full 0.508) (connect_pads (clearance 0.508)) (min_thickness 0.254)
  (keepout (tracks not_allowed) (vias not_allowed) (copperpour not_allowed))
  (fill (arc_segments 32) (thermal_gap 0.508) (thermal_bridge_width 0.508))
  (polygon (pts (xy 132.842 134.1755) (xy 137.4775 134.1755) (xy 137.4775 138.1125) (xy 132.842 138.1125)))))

